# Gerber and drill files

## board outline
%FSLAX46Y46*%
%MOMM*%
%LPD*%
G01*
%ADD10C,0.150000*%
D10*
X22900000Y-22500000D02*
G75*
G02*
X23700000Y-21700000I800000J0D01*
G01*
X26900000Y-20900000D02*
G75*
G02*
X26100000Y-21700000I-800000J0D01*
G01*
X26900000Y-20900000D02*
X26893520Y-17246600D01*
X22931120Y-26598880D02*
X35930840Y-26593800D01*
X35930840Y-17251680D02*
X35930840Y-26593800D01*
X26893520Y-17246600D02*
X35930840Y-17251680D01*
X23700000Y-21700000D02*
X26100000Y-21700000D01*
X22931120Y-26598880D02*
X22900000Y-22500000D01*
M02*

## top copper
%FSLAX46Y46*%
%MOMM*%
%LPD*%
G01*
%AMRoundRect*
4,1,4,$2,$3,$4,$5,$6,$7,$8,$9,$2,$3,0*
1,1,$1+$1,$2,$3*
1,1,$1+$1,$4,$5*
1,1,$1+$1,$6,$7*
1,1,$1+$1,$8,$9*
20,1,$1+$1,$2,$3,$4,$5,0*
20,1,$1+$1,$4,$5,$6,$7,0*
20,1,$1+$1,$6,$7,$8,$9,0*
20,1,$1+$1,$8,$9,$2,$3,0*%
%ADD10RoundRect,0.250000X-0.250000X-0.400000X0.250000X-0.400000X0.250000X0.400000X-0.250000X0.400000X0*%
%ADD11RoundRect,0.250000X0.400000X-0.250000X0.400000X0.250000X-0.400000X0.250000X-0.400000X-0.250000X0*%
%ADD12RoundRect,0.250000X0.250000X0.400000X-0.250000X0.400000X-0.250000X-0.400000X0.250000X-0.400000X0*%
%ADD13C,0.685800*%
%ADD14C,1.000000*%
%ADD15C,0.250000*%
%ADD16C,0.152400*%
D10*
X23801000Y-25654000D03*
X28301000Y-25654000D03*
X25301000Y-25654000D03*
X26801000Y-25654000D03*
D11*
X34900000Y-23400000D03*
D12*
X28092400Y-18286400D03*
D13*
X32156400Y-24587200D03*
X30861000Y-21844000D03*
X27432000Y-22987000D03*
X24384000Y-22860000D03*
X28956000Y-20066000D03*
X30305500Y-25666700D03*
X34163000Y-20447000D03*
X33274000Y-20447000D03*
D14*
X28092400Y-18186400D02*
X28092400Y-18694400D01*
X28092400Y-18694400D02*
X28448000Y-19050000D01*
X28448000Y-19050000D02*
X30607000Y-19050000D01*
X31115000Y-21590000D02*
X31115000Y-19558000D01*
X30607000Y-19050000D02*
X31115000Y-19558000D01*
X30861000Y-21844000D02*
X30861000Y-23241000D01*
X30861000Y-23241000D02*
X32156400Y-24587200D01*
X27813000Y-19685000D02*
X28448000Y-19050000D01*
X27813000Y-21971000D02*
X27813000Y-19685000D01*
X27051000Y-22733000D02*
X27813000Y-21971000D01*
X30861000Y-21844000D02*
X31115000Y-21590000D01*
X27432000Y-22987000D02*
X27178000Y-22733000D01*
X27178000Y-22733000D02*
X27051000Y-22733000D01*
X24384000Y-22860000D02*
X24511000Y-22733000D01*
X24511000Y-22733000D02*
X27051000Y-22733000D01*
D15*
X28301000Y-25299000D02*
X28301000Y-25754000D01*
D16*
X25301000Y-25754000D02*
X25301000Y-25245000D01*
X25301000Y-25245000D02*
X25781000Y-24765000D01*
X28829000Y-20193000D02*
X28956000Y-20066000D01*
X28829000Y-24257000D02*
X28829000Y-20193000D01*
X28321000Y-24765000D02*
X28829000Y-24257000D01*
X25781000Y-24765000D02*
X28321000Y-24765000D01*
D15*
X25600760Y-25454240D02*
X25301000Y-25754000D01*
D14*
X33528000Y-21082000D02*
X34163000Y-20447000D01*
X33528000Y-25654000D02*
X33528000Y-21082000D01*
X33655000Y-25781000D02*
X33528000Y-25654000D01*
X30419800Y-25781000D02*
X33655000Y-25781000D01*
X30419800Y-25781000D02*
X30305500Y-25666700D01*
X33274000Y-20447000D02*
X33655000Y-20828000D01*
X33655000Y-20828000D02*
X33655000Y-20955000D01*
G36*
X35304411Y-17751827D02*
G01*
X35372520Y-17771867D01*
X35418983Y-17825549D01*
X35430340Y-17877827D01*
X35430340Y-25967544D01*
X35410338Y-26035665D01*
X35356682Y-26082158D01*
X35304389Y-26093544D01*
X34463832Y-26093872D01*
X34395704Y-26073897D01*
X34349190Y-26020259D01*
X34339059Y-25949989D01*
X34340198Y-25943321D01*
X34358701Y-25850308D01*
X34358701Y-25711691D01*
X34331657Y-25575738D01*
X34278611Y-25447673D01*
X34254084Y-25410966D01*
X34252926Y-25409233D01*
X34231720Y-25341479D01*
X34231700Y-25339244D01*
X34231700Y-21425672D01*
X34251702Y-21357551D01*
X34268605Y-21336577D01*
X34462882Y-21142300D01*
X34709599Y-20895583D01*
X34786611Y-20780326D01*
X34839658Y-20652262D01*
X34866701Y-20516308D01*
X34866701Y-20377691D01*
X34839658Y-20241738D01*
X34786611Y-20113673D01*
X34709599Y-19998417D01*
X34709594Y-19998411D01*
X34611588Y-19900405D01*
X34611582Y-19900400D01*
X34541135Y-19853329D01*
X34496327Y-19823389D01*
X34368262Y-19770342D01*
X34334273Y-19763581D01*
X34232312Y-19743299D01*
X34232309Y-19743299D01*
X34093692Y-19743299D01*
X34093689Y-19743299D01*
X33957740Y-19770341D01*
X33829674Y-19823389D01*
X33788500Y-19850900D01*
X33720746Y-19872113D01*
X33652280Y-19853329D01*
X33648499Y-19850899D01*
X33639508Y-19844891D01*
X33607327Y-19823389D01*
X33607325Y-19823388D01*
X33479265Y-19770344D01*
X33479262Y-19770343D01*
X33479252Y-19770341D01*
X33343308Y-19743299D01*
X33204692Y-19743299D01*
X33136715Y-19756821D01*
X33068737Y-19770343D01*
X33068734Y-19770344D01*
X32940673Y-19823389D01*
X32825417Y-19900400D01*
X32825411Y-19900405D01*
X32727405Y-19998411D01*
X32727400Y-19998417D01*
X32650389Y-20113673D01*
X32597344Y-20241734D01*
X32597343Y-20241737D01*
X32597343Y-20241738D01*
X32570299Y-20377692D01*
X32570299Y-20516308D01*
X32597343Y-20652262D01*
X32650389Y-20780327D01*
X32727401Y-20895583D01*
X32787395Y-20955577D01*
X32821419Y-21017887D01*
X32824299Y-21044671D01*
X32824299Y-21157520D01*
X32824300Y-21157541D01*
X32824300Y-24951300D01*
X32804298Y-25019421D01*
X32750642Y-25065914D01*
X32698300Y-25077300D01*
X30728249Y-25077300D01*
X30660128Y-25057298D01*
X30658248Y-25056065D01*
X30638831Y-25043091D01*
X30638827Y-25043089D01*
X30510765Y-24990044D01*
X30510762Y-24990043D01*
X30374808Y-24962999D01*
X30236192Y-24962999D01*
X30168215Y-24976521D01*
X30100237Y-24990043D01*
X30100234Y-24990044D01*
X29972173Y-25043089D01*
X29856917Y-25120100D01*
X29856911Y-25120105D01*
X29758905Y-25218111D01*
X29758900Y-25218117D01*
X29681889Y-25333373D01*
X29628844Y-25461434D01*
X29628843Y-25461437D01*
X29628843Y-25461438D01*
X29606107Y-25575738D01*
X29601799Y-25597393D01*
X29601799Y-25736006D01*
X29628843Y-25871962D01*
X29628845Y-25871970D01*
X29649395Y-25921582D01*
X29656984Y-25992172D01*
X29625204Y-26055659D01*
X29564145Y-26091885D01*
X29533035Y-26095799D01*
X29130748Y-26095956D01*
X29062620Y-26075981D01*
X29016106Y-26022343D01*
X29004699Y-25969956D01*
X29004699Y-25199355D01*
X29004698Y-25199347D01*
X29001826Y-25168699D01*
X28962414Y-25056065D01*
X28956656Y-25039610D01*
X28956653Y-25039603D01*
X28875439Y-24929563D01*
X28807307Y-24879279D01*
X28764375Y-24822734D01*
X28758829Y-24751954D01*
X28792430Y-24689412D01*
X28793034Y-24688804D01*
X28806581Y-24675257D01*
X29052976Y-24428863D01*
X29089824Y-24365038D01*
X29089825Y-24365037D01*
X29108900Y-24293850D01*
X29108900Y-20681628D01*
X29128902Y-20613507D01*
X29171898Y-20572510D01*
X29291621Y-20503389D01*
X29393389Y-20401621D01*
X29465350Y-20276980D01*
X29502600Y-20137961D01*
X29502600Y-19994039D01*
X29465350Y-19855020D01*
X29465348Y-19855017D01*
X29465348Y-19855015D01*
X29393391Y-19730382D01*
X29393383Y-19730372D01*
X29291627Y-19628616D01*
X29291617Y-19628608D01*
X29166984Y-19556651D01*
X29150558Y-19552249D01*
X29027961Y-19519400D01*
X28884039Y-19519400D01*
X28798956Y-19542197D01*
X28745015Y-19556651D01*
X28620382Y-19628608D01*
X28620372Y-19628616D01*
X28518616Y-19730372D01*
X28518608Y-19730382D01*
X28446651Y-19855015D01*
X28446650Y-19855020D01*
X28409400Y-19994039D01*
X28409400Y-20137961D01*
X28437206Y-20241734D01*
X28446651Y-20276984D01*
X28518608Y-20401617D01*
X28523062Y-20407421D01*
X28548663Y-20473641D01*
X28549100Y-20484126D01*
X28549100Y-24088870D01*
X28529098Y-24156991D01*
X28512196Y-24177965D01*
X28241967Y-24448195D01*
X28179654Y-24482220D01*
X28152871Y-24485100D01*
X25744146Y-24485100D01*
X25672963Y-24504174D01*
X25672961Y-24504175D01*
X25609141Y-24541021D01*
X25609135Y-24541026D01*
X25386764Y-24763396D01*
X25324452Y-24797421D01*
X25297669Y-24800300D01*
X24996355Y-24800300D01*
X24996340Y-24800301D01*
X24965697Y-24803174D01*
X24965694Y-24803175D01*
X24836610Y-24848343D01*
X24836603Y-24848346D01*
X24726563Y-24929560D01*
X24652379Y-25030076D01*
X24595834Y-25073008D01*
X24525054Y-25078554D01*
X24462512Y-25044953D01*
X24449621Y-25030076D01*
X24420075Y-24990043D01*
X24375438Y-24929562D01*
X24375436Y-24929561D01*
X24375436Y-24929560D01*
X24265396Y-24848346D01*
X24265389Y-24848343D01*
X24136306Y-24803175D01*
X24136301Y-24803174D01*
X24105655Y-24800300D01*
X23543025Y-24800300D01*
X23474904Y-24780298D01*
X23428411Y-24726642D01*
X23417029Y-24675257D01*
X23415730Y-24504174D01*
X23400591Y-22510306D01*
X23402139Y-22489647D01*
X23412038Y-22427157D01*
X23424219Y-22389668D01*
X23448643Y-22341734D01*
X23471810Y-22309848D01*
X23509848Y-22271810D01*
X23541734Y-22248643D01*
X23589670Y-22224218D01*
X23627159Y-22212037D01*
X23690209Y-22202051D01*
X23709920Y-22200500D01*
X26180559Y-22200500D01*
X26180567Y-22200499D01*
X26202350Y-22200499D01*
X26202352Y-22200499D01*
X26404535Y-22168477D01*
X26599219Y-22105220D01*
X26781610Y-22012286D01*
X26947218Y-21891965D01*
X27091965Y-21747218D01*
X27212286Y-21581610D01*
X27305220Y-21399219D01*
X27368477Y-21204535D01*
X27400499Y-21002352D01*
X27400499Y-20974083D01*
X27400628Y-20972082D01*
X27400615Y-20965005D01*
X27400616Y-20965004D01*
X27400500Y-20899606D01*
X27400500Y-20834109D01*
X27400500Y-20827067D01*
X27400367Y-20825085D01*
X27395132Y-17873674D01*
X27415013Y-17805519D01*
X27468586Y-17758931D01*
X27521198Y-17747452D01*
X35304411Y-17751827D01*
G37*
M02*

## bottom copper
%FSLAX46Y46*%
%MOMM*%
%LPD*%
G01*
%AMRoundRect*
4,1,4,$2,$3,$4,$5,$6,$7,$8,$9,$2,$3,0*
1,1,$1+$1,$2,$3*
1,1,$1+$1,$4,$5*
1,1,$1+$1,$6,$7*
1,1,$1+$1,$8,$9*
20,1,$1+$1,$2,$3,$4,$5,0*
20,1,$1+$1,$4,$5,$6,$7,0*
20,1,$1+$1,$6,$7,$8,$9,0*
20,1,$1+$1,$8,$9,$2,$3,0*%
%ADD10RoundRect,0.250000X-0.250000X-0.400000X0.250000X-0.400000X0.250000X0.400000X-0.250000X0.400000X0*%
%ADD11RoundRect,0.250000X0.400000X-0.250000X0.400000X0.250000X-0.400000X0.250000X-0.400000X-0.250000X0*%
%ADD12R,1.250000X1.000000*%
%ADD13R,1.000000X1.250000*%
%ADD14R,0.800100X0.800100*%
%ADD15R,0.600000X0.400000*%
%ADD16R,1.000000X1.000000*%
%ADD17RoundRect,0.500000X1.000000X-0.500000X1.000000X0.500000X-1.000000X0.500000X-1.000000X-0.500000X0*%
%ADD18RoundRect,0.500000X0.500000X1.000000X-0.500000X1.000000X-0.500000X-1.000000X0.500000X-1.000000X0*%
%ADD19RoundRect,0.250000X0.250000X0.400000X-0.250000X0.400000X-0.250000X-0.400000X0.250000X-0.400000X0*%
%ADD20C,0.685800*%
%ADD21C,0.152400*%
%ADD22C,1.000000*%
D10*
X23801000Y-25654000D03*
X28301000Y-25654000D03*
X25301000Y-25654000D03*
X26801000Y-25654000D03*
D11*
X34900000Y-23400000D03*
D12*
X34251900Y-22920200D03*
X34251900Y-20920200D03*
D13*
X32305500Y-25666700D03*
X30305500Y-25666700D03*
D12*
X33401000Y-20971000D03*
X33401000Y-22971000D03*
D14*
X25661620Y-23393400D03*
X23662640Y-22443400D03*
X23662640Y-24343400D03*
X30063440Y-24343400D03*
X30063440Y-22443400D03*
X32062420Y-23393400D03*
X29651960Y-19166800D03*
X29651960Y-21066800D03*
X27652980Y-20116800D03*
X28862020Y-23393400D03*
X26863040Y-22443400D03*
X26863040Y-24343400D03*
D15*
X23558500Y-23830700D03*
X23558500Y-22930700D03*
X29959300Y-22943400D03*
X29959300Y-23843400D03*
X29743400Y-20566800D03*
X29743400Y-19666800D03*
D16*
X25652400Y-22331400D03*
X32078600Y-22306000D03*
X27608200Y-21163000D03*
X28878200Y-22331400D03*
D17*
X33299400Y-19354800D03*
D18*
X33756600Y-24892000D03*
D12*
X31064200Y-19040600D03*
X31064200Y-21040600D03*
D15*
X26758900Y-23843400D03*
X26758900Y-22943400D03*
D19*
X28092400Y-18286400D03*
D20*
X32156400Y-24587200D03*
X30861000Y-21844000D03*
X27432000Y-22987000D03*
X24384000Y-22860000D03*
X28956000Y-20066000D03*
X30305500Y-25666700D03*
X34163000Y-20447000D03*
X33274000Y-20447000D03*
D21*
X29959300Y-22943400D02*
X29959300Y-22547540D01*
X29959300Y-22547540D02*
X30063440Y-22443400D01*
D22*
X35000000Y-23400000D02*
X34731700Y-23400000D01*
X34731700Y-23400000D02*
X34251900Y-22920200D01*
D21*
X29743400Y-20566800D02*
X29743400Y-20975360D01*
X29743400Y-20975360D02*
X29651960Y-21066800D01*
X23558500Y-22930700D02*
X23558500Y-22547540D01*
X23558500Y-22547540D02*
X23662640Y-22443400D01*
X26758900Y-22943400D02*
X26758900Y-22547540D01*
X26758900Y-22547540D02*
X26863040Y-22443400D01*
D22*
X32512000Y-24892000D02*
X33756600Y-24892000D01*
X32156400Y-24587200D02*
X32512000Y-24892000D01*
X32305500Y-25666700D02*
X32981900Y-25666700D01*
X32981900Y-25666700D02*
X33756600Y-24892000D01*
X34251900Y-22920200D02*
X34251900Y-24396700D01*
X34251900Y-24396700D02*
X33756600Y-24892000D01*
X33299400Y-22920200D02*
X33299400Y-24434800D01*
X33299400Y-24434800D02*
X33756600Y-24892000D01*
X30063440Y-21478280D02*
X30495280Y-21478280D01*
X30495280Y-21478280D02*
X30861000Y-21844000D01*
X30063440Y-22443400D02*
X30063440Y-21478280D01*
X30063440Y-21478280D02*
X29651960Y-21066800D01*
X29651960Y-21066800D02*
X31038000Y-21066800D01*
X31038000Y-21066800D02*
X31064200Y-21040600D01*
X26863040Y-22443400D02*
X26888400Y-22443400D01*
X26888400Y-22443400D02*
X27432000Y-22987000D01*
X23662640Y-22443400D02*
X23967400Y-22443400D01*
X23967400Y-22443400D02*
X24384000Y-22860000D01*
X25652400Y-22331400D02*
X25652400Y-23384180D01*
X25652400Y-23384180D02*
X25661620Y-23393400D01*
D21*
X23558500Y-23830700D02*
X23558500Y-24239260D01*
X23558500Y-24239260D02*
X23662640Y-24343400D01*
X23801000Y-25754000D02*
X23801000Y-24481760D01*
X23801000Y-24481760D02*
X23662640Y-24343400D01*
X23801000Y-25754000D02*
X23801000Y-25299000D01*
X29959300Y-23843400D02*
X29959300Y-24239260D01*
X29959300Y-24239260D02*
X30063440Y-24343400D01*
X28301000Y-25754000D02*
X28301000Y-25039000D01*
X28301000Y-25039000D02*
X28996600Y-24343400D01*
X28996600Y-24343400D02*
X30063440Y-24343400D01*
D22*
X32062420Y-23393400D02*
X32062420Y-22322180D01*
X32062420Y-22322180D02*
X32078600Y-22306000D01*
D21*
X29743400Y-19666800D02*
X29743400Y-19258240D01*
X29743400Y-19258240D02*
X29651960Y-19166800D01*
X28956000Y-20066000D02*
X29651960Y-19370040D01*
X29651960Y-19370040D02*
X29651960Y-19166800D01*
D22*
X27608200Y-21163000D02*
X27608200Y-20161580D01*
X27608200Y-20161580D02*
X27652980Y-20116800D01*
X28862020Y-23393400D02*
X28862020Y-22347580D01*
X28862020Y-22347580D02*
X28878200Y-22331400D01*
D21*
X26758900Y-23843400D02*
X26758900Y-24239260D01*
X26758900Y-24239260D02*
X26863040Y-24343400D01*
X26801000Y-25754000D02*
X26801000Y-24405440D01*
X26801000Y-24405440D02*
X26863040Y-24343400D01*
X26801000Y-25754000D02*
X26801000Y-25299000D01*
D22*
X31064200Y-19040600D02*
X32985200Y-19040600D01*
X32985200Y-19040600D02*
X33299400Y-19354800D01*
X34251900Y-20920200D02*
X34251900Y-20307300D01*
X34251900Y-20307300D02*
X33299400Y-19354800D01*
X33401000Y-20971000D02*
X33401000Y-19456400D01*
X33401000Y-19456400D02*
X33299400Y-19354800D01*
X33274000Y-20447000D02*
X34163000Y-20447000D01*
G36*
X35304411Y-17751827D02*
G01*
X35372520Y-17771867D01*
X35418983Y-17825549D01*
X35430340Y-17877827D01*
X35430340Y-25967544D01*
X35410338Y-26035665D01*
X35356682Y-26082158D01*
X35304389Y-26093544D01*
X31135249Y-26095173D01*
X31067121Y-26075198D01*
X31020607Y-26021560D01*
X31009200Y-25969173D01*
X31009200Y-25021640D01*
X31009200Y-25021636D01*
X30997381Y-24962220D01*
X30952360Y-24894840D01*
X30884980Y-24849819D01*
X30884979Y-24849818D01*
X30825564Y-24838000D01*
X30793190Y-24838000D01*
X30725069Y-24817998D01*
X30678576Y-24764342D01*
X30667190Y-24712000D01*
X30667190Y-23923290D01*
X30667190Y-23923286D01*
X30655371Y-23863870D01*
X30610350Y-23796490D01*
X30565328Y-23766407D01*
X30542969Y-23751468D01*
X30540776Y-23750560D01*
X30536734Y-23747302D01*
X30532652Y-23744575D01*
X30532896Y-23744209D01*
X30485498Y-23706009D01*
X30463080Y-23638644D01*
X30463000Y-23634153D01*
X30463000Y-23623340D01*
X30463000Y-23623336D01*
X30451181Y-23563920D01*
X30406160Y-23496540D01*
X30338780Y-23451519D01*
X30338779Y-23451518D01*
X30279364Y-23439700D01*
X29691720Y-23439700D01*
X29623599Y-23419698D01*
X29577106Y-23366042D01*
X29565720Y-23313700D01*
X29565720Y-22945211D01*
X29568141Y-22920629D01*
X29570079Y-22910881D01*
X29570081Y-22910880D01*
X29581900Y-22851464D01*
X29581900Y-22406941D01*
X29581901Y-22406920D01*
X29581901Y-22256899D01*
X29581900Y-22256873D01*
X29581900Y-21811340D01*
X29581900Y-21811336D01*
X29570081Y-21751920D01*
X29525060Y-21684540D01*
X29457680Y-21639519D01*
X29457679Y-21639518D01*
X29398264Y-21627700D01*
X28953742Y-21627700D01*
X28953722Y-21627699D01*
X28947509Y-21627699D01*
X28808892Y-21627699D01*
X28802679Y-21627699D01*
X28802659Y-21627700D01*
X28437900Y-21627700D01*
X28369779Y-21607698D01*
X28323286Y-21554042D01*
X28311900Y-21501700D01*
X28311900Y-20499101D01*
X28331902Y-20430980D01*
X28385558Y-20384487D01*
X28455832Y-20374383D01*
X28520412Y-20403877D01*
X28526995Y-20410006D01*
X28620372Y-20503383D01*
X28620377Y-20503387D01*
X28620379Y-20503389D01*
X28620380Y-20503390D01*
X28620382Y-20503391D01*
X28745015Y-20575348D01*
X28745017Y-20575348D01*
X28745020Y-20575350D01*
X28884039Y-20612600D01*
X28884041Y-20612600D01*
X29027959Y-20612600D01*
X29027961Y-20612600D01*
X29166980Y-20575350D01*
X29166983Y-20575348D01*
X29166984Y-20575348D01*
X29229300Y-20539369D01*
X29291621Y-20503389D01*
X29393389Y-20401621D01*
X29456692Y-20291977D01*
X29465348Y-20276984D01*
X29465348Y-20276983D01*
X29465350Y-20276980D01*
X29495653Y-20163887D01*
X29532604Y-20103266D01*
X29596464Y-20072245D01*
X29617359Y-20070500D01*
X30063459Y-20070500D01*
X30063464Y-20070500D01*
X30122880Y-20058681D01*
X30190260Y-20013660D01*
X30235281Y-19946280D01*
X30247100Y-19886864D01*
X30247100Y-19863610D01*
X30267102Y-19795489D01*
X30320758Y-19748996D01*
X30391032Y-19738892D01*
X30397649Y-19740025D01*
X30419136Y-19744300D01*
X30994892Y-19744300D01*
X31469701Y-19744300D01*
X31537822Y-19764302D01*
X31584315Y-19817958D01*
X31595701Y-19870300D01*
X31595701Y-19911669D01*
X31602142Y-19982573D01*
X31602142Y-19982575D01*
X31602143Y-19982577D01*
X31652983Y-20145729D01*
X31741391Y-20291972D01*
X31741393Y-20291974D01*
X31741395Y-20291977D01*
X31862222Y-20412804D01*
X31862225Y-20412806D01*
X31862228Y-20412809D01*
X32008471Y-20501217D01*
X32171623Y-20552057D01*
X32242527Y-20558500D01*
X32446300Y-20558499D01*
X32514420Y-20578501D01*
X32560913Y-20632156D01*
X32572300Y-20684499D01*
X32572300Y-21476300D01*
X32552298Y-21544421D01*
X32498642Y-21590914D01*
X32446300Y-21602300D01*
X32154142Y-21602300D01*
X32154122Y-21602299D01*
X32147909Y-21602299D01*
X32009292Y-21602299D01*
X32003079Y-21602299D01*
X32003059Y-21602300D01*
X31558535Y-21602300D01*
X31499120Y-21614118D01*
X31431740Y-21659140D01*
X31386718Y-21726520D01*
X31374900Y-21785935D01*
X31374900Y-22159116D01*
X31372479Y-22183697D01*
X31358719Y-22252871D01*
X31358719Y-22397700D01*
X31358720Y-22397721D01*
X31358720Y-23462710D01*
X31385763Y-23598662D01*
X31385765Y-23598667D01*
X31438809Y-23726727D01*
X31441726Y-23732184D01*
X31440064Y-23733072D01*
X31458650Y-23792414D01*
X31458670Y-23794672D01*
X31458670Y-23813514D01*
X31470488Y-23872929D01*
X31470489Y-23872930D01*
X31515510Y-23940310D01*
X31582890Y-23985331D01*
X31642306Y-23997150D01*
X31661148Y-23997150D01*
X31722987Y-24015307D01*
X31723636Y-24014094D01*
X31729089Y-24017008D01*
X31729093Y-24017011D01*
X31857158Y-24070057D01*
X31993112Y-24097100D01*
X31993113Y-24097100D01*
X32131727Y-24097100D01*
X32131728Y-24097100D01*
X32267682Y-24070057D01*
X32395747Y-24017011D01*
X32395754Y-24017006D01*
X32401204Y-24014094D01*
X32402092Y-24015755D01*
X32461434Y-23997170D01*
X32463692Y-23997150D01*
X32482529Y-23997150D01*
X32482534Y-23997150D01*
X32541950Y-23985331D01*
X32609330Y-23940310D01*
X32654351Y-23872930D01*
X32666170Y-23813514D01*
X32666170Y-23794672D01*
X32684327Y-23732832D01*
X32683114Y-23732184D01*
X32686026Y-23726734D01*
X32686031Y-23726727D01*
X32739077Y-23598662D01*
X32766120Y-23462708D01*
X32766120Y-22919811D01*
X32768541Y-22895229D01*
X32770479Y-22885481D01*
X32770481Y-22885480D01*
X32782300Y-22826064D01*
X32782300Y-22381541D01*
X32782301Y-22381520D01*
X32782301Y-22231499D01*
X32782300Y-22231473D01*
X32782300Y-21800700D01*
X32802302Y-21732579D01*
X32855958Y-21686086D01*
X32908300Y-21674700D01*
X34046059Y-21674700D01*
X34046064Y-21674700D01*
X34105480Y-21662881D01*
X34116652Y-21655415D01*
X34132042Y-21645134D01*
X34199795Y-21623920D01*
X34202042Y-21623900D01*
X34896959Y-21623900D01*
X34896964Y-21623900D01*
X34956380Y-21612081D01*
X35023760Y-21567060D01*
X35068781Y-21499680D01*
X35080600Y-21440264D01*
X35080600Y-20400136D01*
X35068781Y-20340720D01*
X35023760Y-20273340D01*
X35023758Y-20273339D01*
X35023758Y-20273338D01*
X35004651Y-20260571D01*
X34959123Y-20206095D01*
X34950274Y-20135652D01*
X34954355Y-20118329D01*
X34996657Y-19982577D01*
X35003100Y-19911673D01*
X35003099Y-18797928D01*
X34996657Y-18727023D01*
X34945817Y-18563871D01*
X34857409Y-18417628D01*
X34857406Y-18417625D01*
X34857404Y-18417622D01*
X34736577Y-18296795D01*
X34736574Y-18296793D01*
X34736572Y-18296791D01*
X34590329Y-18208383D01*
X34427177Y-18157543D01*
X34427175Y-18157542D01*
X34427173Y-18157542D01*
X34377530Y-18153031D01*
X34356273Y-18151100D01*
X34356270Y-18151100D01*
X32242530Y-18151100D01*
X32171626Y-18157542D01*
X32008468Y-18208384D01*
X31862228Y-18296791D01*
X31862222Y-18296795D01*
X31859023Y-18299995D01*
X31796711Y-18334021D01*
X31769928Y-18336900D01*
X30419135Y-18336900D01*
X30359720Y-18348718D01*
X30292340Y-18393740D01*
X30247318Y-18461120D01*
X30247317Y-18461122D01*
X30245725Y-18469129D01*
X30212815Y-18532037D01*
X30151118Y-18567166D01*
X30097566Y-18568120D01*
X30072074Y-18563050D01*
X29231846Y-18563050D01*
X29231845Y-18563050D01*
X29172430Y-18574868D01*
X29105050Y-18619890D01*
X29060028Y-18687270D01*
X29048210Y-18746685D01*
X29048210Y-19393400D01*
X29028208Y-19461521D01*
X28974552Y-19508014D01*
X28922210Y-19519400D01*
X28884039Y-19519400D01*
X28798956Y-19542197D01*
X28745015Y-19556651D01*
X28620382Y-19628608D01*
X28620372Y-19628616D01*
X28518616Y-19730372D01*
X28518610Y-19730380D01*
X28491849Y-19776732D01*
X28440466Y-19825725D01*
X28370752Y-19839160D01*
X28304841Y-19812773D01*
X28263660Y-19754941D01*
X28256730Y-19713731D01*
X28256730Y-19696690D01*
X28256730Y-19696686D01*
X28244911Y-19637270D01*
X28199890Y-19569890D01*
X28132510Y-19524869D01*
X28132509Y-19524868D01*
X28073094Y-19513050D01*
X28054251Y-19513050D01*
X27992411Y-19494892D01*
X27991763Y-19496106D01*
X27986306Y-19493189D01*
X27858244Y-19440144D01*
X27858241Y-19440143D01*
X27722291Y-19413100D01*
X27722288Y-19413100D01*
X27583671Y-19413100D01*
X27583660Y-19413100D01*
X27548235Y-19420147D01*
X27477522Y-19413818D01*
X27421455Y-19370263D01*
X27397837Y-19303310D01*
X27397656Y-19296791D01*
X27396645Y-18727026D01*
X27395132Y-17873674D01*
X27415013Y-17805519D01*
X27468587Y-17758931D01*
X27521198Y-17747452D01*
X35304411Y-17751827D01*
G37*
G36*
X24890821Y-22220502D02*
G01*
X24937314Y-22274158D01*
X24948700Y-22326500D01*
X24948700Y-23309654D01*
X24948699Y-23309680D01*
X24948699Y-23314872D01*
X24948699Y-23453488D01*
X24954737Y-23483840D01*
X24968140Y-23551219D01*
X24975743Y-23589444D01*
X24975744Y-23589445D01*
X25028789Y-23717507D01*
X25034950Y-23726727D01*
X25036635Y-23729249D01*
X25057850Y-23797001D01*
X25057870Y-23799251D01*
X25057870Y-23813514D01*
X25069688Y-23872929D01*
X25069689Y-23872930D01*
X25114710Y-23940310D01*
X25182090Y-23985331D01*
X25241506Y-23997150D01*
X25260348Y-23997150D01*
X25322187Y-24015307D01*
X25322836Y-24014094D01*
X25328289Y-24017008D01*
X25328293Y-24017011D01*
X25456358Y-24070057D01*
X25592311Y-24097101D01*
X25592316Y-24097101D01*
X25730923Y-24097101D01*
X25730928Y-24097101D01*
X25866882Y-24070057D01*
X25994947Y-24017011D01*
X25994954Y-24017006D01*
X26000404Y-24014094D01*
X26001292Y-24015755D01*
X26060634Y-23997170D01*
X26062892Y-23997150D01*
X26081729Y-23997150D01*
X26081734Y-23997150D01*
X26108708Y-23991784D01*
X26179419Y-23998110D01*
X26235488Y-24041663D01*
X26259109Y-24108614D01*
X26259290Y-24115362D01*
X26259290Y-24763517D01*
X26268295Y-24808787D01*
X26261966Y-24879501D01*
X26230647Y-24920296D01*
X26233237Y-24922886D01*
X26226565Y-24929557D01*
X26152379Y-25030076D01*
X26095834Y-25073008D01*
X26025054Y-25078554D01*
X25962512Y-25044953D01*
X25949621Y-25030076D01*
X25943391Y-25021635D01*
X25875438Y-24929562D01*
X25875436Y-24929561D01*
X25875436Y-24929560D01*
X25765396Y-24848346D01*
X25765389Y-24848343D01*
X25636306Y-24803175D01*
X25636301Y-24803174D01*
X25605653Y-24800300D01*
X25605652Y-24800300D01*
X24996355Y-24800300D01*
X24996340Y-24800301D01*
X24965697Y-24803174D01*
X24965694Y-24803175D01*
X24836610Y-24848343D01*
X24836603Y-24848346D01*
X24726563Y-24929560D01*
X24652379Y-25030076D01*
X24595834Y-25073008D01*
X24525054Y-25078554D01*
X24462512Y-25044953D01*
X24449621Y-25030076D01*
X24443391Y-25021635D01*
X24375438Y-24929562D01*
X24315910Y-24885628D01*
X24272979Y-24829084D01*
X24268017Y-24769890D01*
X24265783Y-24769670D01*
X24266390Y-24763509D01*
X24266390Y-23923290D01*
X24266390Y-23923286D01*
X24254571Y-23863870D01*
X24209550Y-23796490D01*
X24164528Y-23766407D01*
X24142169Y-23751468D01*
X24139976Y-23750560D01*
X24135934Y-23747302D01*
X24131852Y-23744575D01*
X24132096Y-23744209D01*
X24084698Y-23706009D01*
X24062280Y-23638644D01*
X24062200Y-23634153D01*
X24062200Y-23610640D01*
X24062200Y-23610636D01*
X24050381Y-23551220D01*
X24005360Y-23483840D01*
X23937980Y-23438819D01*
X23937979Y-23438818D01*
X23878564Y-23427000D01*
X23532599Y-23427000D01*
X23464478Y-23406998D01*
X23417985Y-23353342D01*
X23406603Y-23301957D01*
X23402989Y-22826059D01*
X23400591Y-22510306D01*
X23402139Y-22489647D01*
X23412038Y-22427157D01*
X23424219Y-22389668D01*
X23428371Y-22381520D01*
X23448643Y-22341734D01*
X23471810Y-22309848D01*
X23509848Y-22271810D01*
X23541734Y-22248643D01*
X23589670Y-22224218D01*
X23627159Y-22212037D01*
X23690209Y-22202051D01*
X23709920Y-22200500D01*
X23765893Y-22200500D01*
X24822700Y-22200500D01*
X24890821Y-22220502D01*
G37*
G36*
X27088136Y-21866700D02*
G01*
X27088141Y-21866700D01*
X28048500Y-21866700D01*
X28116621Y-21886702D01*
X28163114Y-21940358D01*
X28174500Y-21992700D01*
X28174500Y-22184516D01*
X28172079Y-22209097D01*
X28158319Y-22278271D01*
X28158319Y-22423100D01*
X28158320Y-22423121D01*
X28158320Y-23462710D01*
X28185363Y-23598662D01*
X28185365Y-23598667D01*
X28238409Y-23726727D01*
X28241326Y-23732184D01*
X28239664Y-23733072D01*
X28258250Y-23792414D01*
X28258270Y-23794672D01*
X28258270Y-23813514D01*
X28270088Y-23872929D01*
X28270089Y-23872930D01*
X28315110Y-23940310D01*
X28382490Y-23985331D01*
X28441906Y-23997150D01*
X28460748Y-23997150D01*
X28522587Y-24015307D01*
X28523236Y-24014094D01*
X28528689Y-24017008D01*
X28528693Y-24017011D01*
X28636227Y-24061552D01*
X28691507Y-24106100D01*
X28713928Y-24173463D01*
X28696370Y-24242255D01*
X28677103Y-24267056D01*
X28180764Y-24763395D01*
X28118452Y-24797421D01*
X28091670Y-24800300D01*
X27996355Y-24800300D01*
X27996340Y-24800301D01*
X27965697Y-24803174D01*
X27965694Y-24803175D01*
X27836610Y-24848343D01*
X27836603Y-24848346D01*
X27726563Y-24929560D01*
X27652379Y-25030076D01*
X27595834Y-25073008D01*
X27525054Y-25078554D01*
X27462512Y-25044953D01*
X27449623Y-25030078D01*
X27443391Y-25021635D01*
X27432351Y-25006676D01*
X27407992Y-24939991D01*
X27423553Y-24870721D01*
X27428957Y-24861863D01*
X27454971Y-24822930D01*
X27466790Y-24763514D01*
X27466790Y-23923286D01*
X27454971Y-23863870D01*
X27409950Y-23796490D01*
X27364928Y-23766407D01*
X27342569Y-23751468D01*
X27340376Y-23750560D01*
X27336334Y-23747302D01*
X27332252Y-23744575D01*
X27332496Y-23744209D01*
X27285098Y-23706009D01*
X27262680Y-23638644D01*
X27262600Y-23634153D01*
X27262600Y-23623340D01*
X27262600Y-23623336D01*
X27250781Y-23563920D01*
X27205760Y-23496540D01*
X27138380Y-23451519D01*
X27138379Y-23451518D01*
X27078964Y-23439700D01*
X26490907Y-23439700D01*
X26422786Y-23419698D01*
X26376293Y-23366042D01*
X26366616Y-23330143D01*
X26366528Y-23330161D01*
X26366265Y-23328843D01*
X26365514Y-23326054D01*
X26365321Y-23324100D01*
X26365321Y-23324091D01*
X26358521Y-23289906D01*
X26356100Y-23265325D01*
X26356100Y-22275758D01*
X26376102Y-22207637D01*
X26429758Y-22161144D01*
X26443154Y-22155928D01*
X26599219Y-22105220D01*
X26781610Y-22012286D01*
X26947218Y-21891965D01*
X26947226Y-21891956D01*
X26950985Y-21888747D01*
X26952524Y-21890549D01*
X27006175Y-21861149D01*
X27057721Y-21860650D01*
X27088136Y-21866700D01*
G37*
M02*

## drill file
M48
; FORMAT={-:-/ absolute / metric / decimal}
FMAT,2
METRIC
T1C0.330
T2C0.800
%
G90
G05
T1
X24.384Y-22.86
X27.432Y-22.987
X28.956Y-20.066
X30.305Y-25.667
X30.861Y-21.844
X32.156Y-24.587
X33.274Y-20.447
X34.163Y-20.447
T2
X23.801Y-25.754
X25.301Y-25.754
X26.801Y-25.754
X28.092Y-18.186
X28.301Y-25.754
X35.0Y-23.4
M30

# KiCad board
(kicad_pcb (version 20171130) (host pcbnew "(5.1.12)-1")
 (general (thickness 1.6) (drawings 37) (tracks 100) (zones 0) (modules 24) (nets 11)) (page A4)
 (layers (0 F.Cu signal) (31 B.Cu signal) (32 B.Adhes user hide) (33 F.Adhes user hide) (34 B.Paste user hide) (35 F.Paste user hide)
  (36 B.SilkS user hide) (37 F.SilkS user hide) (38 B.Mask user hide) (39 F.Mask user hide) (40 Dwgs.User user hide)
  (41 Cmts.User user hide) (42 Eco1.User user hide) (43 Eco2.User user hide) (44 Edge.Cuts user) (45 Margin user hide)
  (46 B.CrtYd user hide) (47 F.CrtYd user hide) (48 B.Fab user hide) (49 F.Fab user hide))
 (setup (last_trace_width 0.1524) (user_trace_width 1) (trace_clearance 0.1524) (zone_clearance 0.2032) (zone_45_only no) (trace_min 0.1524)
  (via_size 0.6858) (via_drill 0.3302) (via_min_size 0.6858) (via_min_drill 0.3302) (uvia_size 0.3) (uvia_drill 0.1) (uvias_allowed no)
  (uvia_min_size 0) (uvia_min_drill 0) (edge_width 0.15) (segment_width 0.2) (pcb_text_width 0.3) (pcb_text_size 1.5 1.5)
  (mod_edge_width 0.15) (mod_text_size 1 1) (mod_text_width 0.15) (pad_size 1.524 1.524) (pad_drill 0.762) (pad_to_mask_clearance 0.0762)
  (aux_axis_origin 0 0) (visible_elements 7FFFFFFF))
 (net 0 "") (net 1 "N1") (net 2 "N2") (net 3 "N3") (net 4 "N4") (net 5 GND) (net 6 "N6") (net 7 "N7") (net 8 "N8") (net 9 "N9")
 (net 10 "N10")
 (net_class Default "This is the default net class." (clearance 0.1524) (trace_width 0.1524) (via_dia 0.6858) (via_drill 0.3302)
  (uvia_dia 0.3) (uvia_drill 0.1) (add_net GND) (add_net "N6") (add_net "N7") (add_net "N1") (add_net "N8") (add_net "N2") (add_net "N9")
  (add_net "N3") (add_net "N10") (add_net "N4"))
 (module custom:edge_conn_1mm (layer F.Cu) (at 23.801 25.754)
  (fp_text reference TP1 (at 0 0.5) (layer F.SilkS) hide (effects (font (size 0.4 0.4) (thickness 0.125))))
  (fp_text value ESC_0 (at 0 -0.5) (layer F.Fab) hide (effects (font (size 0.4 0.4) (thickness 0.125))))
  (pad 1 thru_hole roundrect (at 0 0) (size 1 1.3) (drill 0.8 (offset 0 -0.1)) (layers *.Cu *.Mask) (roundrect_rratio 0.25) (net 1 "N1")))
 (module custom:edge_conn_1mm (layer F.Cu) (at 28.301 25.754)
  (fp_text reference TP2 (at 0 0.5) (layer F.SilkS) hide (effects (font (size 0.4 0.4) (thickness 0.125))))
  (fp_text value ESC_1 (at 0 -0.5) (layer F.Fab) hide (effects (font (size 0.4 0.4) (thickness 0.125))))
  (pad 1 thru_hole roundrect (at 0 0) (size 1 1.3) (drill 0.8 (offset 0 -0.1)) (layers *.Cu *.Mask) (roundrect_rratio 0.25) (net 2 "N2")))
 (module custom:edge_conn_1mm (layer F.Cu) (at 25.301 25.754)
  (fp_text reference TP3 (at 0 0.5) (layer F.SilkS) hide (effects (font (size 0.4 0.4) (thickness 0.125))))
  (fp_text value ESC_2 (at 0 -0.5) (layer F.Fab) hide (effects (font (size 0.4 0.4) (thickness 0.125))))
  (pad 1 thru_hole roundrect (at 0 0) (size 1 1.3) (drill 0.8 (offset 0 -0.1)) (layers *.Cu *.Mask) (roundrect_rratio 0.25) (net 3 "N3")))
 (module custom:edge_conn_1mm (layer F.Cu) (at 26.801 25.754)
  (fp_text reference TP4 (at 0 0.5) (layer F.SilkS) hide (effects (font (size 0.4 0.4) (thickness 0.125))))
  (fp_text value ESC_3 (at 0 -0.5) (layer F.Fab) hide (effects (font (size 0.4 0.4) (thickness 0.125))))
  (pad 1 thru_hole roundrect (at 0 0) (size 1 1.3) (drill 0.8 (offset 0 -0.1)) (layers *.Cu *.Mask) (roundrect_rratio 0.25) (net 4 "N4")))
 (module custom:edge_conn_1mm (layer F.Cu) (at 35 23.4 90)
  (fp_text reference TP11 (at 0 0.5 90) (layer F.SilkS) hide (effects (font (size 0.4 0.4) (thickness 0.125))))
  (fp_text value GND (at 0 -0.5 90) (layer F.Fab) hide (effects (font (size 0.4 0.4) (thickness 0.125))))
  (pad 1 thru_hole roundrect (at 0 0 90) (size 1 1.3) (drill 0.8 (offset 0 -0.1)) (layers *.Cu *.Mask) (roundrect_rratio 0.25) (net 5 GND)))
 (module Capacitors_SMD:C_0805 (layer B.Cu) (at 34.2519 21.9202 270)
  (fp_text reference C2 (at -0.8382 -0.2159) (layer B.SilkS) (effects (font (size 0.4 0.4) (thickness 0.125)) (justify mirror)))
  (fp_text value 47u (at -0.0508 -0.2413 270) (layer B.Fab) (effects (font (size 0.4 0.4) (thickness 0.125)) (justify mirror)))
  (pad 2 smd rect (at 1 0 270) (size 1 1.25) (layers B.Cu B.Paste B.Mask) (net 5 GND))
  (pad 1 smd rect (at -1 0 270) (size 1 1.25) (layers B.Cu B.Paste B.Mask) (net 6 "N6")))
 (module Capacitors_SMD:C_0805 (layer B.Cu) (at 31.3055 25.6667)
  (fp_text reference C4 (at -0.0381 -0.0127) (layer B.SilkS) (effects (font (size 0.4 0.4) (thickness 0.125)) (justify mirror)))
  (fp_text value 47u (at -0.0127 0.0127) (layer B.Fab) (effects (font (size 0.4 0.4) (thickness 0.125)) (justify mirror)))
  (pad 2 smd rect (at 1 0) (size 1 1.25) (layers B.Cu B.Paste B.Mask) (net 5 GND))
  (pad 1 smd rect (at -1 0) (size 1 1.25) (layers B.Cu B.Paste B.Mask) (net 6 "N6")))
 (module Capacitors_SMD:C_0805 (layer B.Cu) (at 33.401 21.971 270)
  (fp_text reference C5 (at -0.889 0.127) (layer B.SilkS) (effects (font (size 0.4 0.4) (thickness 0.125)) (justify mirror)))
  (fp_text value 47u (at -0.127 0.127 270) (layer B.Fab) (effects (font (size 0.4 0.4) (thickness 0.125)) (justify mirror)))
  (pad 1 smd rect (at -1 0 270) (size 1 1.25) (layers B.Cu B.Paste B.Mask) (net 6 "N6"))
  (pad 2 smd rect (at 1 0 270) (size 1 1.25) (layers B.Cu B.Paste B.Mask) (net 5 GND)))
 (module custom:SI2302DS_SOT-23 (layer B.Cu) (at 24.6634 23.3934 90)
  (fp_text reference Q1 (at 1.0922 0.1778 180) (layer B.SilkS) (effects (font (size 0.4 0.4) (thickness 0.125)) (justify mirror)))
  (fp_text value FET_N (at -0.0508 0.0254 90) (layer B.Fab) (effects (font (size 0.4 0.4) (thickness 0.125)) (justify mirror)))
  (pad D smd rect (at 0 0.99822 90) (size 0.8001 0.8001) (layers B.Cu B.Paste B.Mask) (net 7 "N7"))
  (pad S smd rect (at 0.95 -1.00076 90) (size 0.8001 0.8001) (layers B.Cu B.Paste B.Mask) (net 5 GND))
  (pad G smd rect (at -0.95 -1.00076 90) (size 0.8001 0.8001) (layers B.Cu B.Paste B.Mask) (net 1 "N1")))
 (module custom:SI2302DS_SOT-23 (layer B.Cu) (at 31.0642 23.3934 90)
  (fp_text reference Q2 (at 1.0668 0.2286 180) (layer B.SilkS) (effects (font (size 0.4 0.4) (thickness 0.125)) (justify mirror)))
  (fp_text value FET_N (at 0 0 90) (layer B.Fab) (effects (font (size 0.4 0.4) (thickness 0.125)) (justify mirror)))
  (pad G smd rect (at -0.95 -1.00076 90) (size 0.8001 0.8001) (layers B.Cu B.Paste B.Mask) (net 2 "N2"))
  (pad S smd rect (at 0.95 -1.00076 90) (size 0.8001 0.8001) (layers B.Cu B.Paste B.Mask) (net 5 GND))
  (pad D smd rect (at 0 0.99822 90) (size 0.8001 0.8001) (layers B.Cu B.Paste B.Mask) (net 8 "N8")))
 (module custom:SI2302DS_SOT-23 (layer B.Cu) (at 28.6512 20.1168 270)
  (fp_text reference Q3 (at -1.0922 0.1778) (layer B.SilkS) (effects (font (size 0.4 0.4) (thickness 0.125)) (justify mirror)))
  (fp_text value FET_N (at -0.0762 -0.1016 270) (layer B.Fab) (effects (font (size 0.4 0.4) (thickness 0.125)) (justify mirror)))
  (pad G smd rect (at -0.95 -1.00076 270) (size 0.8001 0.8001) (layers B.Cu B.Paste B.Mask) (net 3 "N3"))
  (pad S smd rect (at 0.95 -1.00076 270) (size 0.8001 0.8001) (layers B.Cu B.Paste B.Mask) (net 5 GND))
  (pad D smd rect (at 0 0.99822 270) (size 0.8001 0.8001) (layers B.Cu B.Paste B.Mask) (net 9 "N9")))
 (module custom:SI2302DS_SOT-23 (layer B.Cu) (at 27.8638 23.3934 90)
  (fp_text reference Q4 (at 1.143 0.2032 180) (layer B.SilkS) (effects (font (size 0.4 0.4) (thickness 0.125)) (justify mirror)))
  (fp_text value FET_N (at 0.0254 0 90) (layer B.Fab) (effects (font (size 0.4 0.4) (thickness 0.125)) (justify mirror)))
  (pad D smd rect (at 0 0.99822 90) (size 0.8001 0.8001) (layers B.Cu B.Paste B.Mask) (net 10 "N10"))
  (pad S smd rect (at 0.95 -1.00076 90) (size 0.8001 0.8001) (layers B.Cu B.Paste B.Mask) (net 5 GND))
  (pad G smd rect (at -0.95 -1.00076 90) (size 0.8001 0.8001) (layers B.Cu B.Paste B.Mask) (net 4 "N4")))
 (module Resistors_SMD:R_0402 (layer B.Cu) (at 23.5585 23.3807 90)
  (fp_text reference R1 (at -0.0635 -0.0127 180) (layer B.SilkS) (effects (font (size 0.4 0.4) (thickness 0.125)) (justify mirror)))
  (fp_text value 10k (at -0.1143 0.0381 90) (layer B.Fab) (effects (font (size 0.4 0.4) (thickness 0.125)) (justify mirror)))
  (pad 1 smd rect (at -0.45 0 90) (size 0.4 0.6) (layers B.Cu B.Paste B.Mask) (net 1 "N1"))
  (pad 2 smd rect (at 0.45 0 90) (size 0.4 0.6) (layers B.Cu B.Paste B.Mask) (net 5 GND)))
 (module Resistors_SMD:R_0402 (layer B.Cu) (at 29.9593 23.3934 90)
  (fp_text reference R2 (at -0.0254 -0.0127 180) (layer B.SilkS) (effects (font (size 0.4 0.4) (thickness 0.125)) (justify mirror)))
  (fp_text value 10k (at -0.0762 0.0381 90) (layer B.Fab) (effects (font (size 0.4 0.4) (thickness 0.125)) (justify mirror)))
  (pad 2 smd rect (at 0.45 0 90) (size 0.4 0.6) (layers B.Cu B.Paste B.Mask) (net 5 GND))
  (pad 1 smd rect (at -0.45 0 90) (size 0.4 0.6) (layers B.Cu B.Paste B.Mask) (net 2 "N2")))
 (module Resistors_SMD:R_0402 (layer B.Cu) (at 29.7434 20.1168 270)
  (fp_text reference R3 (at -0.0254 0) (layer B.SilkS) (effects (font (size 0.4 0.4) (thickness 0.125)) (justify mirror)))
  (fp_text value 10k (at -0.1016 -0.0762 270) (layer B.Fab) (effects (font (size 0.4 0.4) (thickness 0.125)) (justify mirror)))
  (pad 2 smd rect (at 0.45 0 270) (size 0.4 0.6) (layers B.Cu B.Paste B.Mask) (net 5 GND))
  (pad 1 smd rect (at -0.45 0 270) (size 0.4 0.6) (layers B.Cu B.Paste B.Mask) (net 3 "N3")))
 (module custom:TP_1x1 (layer B.Cu) (at 25.5524 22.6314)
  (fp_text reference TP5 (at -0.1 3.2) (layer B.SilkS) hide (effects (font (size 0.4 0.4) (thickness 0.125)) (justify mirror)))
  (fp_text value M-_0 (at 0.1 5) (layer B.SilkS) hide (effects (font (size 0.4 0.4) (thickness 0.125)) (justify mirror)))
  (pad 1 smd rect (at 0.1 -0.3) (size 1 1) (layers B.Cu B.Mask) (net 7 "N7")))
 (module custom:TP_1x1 (layer B.Cu) (at 31.9786 22.606)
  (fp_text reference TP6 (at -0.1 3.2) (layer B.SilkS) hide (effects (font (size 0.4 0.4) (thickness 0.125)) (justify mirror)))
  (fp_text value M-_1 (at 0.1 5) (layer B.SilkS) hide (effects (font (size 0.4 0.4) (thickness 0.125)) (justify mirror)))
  (pad 1 smd rect (at 0.1 -0.3) (size 1 1) (layers B.Cu B.Mask) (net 8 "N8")))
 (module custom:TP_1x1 (layer B.Cu) (at 27.5082 21.463)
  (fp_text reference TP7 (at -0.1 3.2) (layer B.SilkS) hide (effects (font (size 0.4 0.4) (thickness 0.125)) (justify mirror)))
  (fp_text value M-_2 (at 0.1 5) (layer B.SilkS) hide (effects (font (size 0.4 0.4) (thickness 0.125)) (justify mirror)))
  (pad 1 smd rect (at 0.1 -0.3) (size 1 1) (layers B.Cu B.Mask) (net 9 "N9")))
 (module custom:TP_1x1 (layer B.Cu) (at 28.7782 22.6314)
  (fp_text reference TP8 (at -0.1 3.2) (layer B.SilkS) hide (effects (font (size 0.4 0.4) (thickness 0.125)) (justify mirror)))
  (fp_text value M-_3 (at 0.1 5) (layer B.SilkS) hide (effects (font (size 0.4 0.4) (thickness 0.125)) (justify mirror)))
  (pad 1 smd rect (at 0.1 -0.3) (size 1 1) (layers B.Cu B.Mask) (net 10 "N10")))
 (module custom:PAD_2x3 (layer B.Cu) (at 33.2994 19.3548 90)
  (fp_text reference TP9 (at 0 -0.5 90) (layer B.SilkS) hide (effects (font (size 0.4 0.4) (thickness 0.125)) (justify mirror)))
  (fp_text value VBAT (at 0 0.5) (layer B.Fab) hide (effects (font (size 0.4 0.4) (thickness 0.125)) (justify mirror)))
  (pad 1 smd roundrect (at 0 0 90) (size 2 3) (layers B.Cu B.Mask) (roundrect_rratio 0.25) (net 6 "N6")))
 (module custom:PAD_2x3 (layer B.Cu) (at 33.7566 24.892 180)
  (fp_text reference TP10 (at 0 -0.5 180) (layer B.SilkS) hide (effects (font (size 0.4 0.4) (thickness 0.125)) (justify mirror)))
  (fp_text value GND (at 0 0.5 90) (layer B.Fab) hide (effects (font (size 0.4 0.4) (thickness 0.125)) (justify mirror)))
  (pad 1 smd roundrect (at 0 0 180) (size 2 3) (layers B.Cu B.Mask) (roundrect_rratio 0.25) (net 5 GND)))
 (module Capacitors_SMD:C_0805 (layer B.Cu) (at 31.0642 20.0406 270)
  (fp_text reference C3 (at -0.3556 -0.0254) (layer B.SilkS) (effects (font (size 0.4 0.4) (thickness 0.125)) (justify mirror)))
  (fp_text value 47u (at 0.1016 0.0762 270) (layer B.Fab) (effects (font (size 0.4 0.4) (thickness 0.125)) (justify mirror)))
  (pad 1 smd rect (at -1 0 270) (size 1 1.25) (layers B.Cu B.Paste B.Mask) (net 6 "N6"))
  (pad 2 smd rect (at 1 0 270) (size 1 1.25) (layers B.Cu B.Paste B.Mask) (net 5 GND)))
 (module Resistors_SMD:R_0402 (layer B.Cu) (at 26.7589 23.3934 90)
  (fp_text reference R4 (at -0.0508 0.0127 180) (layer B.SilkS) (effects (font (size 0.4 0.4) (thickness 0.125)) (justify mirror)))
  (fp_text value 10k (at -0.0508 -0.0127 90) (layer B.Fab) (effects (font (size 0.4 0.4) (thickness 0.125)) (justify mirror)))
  (pad 1 smd rect (at -0.45 0 90) (size 0.4 0.6) (layers B.Cu B.Paste B.Mask) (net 4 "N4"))
  (pad 2 smd rect (at 0.45 0 90) (size 0.4 0.6) (layers B.Cu B.Paste B.Mask) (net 5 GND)))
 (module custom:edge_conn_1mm (layer F.Cu) (at 28.0924 18.1864 180)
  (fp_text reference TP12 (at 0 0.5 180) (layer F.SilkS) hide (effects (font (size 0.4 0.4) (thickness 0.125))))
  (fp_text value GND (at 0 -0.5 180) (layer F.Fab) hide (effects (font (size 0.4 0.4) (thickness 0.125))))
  (pad 1 thru_hole roundrect (at 0 0 180) (size 1 1.3) (drill 0.8 (offset 0 -0.1)) (layers *.Cu *.Mask) (roundrect_rratio 0.25) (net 5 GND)))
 (gr_arc (start 23.7 22.5) (end 22.9 22.5) (angle 90) (layer Edge.Cuts) (width 0.15))
 (gr_arc (start 26.1 20.9) (end 26.9 20.9) (angle 90) (layer Edge.Cuts) (width 0.15))
 (gr_line (start 26.9 20.9) (end 26.89352 17.2466) (angle 90) (layer Edge.Cuts) (width 0.15))
 (gr_line (start 22.93112 26.59888) (end 35.93084 26.5938) (angle 90) (layer Edge.Cuts) (width 0.15))
 (gr_line (start 35.93084 17.25168) (end 35.93084 26.5938) (angle 90) (layer Edge.Cuts) (width 0.15))
 (gr_line (start 26.89352 17.2466) (end 35.93084 17.25168) (angle 90) (layer Edge.Cuts) (width 0.15))
 (gr_line (start 23.7 21.7) (end 26.1 21.7) (angle 90) (layer Edge.Cuts) (width 0.15))
 (gr_line (start 22.93112 26.59888) (end 22.9 22.5) (angle 90) (layer Edge.Cuts) (width 0.15))
 (segment (start 28.0924 18.1864) (end 28.0924 18.6944) (width 1) (layer F.Cu) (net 5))
 (segment (start 28.0924 18.6944) (end 28.448 19.05) (width 1) (layer F.Cu) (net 5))
 (segment (start 29.9593 22.9434) (end 29.9593 22.54754) (width 0.1524) (layer B.Cu) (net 5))
 (segment (start 29.9593 22.54754) (end 30.06344 22.4434) (width 0.1524) (layer B.Cu) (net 5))
 (segment (start 35 23.4) (end 34.7317 23.4) (width 1) (layer B.Cu) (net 5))
 (segment (start 34.7317 23.4) (end 34.2519 22.9202) (width 1) (layer B.Cu) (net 5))
 (segment (start 28.448 19.05) (end 30.607 19.05) (width 1) (layer F.Cu) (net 5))
 (segment (start 31.115 21.59) (end 31.115 19.558) (width 1) (layer F.Cu) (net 5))
 (segment (start 30.607 19.05) (end 31.115 19.558) (width 1) (layer F.Cu) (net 5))
 (segment (start 29.7434 20.5668) (end 29.7434 20.97536) (width 0.1524) (layer B.Cu) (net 5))
 (segment (start 29.7434 20.97536) (end 29.65196 21.0668) (width 0.1524) (layer B.Cu) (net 5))
 (segment (start 23.5585 22.9307) (end 23.5585 22.54754) (width 0.1524) (layer B.Cu) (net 5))
 (segment (start 23.5585 22.54754) (end 23.66264 22.4434) (width 0.1524) (layer B.Cu) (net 5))
 (segment (start 26.7589 22.9434) (end 26.7589 22.54754) (width 0.1524) (layer B.Cu) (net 5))
 (segment (start 26.7589 22.54754) (end 26.86304 22.4434) (width 0.1524) (layer B.Cu) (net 5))
 (segment (start 30.861 21.844) (end 30.861 23.241) (width 1) (layer F.Cu) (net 5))
 (segment (start 32.512 24.892) (end 33.7566 24.892) (width 1) (layer B.Cu) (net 5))
 (segment (start 32.1564 24.5872) (end 32.512 24.892) (width 1) (layer B.Cu) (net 5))
 (via (at 32.1564 24.5872) (size 0.6858) (drill 0.3302) (layers F.Cu B.Cu) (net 5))
 (segment (start 30.861 23.241) (end 32.1564 24.5872) (width 1) (layer F.Cu) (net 5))
 (segment (start 32.3055 25.6667) (end 32.9819 25.6667) (width 1) (layer B.Cu) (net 5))
 (segment (start 32.9819 25.6667) (end 33.7566 24.892) (width 1) (layer B.Cu) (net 5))
 (segment (start 34.2519 22.9202) (end 34.2519 24.3967) (width 1) (layer B.Cu) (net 5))
 (segment (start 34.2519 24.3967) (end 33.7566 24.892) (width 1) (layer B.Cu) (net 5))
 (segment (start 33.2994 22.9202) (end 33.2994 24.4348) (width 1) (layer B.Cu) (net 5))
 (segment (start 33.2994 24.4348) (end 33.7566 24.892) (width 1) (layer B.Cu) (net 5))
 (segment (start 30.06344 21.47828) (end 30.49528 21.47828) (width 1) (layer B.Cu) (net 5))
 (segment (start 30.49528 21.47828) (end 30.861 21.844) (width 1) (layer B.Cu) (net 5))
 (segment (start 27.813 19.685) (end 28.448 19.05) (width 1) (layer F.Cu) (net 5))
 (segment (start 27.813 21.971) (end 27.813 19.685) (width 1) (layer F.Cu) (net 5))
 (segment (start 27.051 22.733) (end 27.813 21.971) (width 1) (layer F.Cu) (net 5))
 (segment (start 30.861 21.844) (end 31.115 21.59) (width 1) (layer F.Cu) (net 5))
 (via (at 30.861 21.844) (size 0.6858) (drill 0.3302) (layers F.Cu B.Cu) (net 5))
 (segment (start 30.06344 22.4434) (end 30.06344 21.47828) (width 1) (layer B.Cu) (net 5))
 (segment (start 30.06344 21.47828) (end 29.65196 21.0668) (width 1) (layer B.Cu) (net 5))
 (segment (start 29.65196 21.0668) (end 31.038 21.0668) (width 1) (layer B.Cu) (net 5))
 (segment (start 31.038 21.0668) (end 31.0642 21.0406) (width 1) (layer B.Cu) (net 5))
 (segment (start 26.86304 22.4434) (end 26.8884 22.4434) (width 1) (layer B.Cu) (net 5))
 (segment (start 26.8884 22.4434) (end 27.432 22.987) (width 1) (layer B.Cu) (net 5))
 (via (at 27.432 22.987) (size 0.6858) (drill 0.3302) (layers F.Cu B.Cu) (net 5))
 (segment (start 27.432 22.987) (end 27.178 22.733) (width 1) (layer F.Cu) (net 5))
 (segment (start 27.178 22.733) (end 27.051 22.733) (width 1) (layer F.Cu) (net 5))
 (segment (start 23.66264 22.4434) (end 23.9674 22.4434) (width 1) (layer B.Cu) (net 5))
 (segment (start 23.9674 22.4434) (end 24.384 22.86) (width 1) (layer B.Cu) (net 5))
 (via (at 24.384 22.86) (size 0.6858) (drill 0.3302) (layers F.Cu B.Cu) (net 5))
 (segment (start 24.384 22.86) (end 24.511 22.733) (width 1) (layer F.Cu) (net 5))
 (segment (start 24.511 22.733) (end 27.051 22.733) (width 1) (layer F.Cu) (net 5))
 (segment (start 25.6524 22.3314) (end 25.6524 23.38418) (width 1) (layer B.Cu) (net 7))
 (segment (start 25.6524 23.38418) (end 25.66162 23.3934) (width 1) (layer B.Cu) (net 7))
 (segment (start 23.5585 23.8307) (end 23.5585 24.23926) (width 0.1524) (layer B.Cu) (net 1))
 (segment (start 23.5585 24.23926) (end 23.66264 24.3434) (width 0.1524) (layer B.Cu) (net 1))
 (segment (start 23.801 25.754) (end 23.801 24.48176) (width 0.1524) (layer B.Cu) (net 1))
 (segment (start 23.801 24.48176) (end 23.66264 24.3434) (width 0.1524) (layer B.Cu) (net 1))
 (segment (start 23.801 25.754) (end 23.801 25.299) (width 0.1524) (layer B.Cu) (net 1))
 (segment (start 29.9593 23.8434) (end 29.9593 24.23926) (width 0.1524) (layer B.Cu) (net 2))
 (segment (start 29.9593 24.23926) (end 30.06344 24.3434) (width 0.1524) (layer B.Cu) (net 2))
 (segment (start 28.301 25.754) (end 28.301 25.039) (width 0.1524) (layer B.Cu) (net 2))
 (segment (start 28.301 25.039) (end 28.9966 24.3434) (width 0.1524) (layer B.Cu) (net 2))
 (segment (start 28.9966 24.3434) (end 30.06344 24.3434) (width 0.1524) (layer B.Cu) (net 2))
 (segment (start 28.301 25.299) (end 28.301 25.754) (width 0.25) (layer F.Cu) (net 2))
 (segment (start 32.06242 23.3934) (end 32.06242 22.32218) (width 1) (layer B.Cu) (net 8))
 (segment (start 32.06242 22.32218) (end 32.0786 22.306) (width 1) (layer B.Cu) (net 8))
 (segment (start 29.7434 19.6668) (end 29.7434 19.25824) (width 0.1524) (layer B.Cu) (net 3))
 (segment (start 29.7434 19.25824) (end 29.65196 19.1668) (width 0.1524) (layer B.Cu) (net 3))
 (segment (start 25.301 25.754) (end 25.301 25.245) (width 0.1524) (layer F.Cu) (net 3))
 (segment (start 25.301 25.245) (end 25.781 24.765) (width 0.1524) (layer F.Cu) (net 3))
 (segment (start 28.956 20.066) (end 29.65196 19.37004) (width 0.1524) (layer B.Cu) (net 3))
 (via (at 28.956 20.066) (size 0.6858) (drill 0.3302) (layers F.Cu B.Cu) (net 3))
 (segment (start 28.829 20.193) (end 28.956 20.066) (width 0.1524) (layer F.Cu) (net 3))
 (segment (start 28.829 24.257) (end 28.829 20.193) (width 0.1524) (layer F.Cu) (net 3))
 (segment (start 28.321 24.765) (end 28.829 24.257) (width 0.1524) (layer F.Cu) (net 3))
 (segment (start 25.781 24.765) (end 28.321 24.765) (width 0.1524) (layer F.Cu) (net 3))
 (segment (start 29.65196 19.37004) (end 29.65196 19.1668) (width 0.1524) (layer B.Cu) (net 3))
 (segment (start 25.60076 25.45424) (end 25.301 25.754) (width 0.25) (layer F.Cu) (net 3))
 (segment (start 27.6082 21.163) (end 27.6082 20.16158) (width 1) (layer B.Cu) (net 9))
 (segment (start 27.6082 20.16158) (end 27.65298 20.1168) (width 1) (layer B.Cu) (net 9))
 (segment (start 28.86202 23.3934) (end 28.86202 22.34758) (width 1) (layer B.Cu) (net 10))
 (segment (start 28.86202 22.34758) (end 28.8782 22.3314) (width 1) (layer B.Cu) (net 10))
 (segment (start 26.7589 23.8434) (end 26.7589 24.23926) (width 0.1524) (layer B.Cu) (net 4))
 (segment (start 26.7589 24.23926) (end 26.86304 24.3434) (width 0.1524) (layer B.Cu) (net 4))
 (segment (start 26.801 25.754) (end 26.801 24.40544) (width 0.1524) (layer B.Cu) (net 4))
 (segment (start 26.801 24.40544) (end 26.86304 24.3434) (width 0.1524) (layer B.Cu) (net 4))
 (segment (start 26.801 25.754) (end 26.801 25.299) (width 0.1524) (layer B.Cu) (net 4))
 (segment (start 31.0642 19.0406) (end 32.9852 19.0406) (width 1) (layer B.Cu) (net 6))
 (segment (start 32.9852 19.0406) (end 33.2994 19.3548) (width 1) (layer B.Cu) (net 6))
 (segment (start 34.2519 20.9202) (end 34.2519 20.3073) (width 1) (layer B.Cu) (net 6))
 (segment (start 34.2519 20.3073) (end 33.2994 19.3548) (width 1) (layer B.Cu) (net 6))
 (segment (start 33.401 20.971) (end 33.401 19.4564) (width 1) (layer B.Cu) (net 6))
 (segment (start 33.401 19.4564) (end 33.2994 19.3548) (width 1) (layer B.Cu) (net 6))
 (via (at 30.3055 25.6667) (size 0.6858) (drill 0.3302) (layers F.Cu B.Cu) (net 6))
 (segment (start 33.274 20.447) (end 34.163 20.447) (width 1) (layer B.Cu) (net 6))
 (via (at 34.163 20.447) (size 0.6858) (drill 0.3302) (layers F.Cu B.Cu) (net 6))
 (segment (start 33.528 21.082) (end 34.163 20.447) (width 1) (layer F.Cu) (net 6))
 (segment (start 33.528 25.654) (end 33.528 21.082) (width 1) (layer F.Cu) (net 6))
 (segment (start 33.655 25.781) (end 33.528 25.654) (width 1) (layer F.Cu) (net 6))
 (segment (start 30.4198 25.781) (end 33.655 25.781) (width 1) (layer F.Cu) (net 6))
 (segment (start 30.4198 25.781) (end 30.3055 25.6667) (width 1) (layer F.Cu) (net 6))
 (via (at 33.274 20.447) (size 0.6858) (drill 0.3302) (layers F.Cu B.Cu) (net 6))
 (segment (start 33.274 20.447) (end 33.655 20.828) (width 1) (layer F.Cu) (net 6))
 (segment (start 33.655 20.828) (end 33.655 20.955) (width 1) (layer F.Cu) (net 6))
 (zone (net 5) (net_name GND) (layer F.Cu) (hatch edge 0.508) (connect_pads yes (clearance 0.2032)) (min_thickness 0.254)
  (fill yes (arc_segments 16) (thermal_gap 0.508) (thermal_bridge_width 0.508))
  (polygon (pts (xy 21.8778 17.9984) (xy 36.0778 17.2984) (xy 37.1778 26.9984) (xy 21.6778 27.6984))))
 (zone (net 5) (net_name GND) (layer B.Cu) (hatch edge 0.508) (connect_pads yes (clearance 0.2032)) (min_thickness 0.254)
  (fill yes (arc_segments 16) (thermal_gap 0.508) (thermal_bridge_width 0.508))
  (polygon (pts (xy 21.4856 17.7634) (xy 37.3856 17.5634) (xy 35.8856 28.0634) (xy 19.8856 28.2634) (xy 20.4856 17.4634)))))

